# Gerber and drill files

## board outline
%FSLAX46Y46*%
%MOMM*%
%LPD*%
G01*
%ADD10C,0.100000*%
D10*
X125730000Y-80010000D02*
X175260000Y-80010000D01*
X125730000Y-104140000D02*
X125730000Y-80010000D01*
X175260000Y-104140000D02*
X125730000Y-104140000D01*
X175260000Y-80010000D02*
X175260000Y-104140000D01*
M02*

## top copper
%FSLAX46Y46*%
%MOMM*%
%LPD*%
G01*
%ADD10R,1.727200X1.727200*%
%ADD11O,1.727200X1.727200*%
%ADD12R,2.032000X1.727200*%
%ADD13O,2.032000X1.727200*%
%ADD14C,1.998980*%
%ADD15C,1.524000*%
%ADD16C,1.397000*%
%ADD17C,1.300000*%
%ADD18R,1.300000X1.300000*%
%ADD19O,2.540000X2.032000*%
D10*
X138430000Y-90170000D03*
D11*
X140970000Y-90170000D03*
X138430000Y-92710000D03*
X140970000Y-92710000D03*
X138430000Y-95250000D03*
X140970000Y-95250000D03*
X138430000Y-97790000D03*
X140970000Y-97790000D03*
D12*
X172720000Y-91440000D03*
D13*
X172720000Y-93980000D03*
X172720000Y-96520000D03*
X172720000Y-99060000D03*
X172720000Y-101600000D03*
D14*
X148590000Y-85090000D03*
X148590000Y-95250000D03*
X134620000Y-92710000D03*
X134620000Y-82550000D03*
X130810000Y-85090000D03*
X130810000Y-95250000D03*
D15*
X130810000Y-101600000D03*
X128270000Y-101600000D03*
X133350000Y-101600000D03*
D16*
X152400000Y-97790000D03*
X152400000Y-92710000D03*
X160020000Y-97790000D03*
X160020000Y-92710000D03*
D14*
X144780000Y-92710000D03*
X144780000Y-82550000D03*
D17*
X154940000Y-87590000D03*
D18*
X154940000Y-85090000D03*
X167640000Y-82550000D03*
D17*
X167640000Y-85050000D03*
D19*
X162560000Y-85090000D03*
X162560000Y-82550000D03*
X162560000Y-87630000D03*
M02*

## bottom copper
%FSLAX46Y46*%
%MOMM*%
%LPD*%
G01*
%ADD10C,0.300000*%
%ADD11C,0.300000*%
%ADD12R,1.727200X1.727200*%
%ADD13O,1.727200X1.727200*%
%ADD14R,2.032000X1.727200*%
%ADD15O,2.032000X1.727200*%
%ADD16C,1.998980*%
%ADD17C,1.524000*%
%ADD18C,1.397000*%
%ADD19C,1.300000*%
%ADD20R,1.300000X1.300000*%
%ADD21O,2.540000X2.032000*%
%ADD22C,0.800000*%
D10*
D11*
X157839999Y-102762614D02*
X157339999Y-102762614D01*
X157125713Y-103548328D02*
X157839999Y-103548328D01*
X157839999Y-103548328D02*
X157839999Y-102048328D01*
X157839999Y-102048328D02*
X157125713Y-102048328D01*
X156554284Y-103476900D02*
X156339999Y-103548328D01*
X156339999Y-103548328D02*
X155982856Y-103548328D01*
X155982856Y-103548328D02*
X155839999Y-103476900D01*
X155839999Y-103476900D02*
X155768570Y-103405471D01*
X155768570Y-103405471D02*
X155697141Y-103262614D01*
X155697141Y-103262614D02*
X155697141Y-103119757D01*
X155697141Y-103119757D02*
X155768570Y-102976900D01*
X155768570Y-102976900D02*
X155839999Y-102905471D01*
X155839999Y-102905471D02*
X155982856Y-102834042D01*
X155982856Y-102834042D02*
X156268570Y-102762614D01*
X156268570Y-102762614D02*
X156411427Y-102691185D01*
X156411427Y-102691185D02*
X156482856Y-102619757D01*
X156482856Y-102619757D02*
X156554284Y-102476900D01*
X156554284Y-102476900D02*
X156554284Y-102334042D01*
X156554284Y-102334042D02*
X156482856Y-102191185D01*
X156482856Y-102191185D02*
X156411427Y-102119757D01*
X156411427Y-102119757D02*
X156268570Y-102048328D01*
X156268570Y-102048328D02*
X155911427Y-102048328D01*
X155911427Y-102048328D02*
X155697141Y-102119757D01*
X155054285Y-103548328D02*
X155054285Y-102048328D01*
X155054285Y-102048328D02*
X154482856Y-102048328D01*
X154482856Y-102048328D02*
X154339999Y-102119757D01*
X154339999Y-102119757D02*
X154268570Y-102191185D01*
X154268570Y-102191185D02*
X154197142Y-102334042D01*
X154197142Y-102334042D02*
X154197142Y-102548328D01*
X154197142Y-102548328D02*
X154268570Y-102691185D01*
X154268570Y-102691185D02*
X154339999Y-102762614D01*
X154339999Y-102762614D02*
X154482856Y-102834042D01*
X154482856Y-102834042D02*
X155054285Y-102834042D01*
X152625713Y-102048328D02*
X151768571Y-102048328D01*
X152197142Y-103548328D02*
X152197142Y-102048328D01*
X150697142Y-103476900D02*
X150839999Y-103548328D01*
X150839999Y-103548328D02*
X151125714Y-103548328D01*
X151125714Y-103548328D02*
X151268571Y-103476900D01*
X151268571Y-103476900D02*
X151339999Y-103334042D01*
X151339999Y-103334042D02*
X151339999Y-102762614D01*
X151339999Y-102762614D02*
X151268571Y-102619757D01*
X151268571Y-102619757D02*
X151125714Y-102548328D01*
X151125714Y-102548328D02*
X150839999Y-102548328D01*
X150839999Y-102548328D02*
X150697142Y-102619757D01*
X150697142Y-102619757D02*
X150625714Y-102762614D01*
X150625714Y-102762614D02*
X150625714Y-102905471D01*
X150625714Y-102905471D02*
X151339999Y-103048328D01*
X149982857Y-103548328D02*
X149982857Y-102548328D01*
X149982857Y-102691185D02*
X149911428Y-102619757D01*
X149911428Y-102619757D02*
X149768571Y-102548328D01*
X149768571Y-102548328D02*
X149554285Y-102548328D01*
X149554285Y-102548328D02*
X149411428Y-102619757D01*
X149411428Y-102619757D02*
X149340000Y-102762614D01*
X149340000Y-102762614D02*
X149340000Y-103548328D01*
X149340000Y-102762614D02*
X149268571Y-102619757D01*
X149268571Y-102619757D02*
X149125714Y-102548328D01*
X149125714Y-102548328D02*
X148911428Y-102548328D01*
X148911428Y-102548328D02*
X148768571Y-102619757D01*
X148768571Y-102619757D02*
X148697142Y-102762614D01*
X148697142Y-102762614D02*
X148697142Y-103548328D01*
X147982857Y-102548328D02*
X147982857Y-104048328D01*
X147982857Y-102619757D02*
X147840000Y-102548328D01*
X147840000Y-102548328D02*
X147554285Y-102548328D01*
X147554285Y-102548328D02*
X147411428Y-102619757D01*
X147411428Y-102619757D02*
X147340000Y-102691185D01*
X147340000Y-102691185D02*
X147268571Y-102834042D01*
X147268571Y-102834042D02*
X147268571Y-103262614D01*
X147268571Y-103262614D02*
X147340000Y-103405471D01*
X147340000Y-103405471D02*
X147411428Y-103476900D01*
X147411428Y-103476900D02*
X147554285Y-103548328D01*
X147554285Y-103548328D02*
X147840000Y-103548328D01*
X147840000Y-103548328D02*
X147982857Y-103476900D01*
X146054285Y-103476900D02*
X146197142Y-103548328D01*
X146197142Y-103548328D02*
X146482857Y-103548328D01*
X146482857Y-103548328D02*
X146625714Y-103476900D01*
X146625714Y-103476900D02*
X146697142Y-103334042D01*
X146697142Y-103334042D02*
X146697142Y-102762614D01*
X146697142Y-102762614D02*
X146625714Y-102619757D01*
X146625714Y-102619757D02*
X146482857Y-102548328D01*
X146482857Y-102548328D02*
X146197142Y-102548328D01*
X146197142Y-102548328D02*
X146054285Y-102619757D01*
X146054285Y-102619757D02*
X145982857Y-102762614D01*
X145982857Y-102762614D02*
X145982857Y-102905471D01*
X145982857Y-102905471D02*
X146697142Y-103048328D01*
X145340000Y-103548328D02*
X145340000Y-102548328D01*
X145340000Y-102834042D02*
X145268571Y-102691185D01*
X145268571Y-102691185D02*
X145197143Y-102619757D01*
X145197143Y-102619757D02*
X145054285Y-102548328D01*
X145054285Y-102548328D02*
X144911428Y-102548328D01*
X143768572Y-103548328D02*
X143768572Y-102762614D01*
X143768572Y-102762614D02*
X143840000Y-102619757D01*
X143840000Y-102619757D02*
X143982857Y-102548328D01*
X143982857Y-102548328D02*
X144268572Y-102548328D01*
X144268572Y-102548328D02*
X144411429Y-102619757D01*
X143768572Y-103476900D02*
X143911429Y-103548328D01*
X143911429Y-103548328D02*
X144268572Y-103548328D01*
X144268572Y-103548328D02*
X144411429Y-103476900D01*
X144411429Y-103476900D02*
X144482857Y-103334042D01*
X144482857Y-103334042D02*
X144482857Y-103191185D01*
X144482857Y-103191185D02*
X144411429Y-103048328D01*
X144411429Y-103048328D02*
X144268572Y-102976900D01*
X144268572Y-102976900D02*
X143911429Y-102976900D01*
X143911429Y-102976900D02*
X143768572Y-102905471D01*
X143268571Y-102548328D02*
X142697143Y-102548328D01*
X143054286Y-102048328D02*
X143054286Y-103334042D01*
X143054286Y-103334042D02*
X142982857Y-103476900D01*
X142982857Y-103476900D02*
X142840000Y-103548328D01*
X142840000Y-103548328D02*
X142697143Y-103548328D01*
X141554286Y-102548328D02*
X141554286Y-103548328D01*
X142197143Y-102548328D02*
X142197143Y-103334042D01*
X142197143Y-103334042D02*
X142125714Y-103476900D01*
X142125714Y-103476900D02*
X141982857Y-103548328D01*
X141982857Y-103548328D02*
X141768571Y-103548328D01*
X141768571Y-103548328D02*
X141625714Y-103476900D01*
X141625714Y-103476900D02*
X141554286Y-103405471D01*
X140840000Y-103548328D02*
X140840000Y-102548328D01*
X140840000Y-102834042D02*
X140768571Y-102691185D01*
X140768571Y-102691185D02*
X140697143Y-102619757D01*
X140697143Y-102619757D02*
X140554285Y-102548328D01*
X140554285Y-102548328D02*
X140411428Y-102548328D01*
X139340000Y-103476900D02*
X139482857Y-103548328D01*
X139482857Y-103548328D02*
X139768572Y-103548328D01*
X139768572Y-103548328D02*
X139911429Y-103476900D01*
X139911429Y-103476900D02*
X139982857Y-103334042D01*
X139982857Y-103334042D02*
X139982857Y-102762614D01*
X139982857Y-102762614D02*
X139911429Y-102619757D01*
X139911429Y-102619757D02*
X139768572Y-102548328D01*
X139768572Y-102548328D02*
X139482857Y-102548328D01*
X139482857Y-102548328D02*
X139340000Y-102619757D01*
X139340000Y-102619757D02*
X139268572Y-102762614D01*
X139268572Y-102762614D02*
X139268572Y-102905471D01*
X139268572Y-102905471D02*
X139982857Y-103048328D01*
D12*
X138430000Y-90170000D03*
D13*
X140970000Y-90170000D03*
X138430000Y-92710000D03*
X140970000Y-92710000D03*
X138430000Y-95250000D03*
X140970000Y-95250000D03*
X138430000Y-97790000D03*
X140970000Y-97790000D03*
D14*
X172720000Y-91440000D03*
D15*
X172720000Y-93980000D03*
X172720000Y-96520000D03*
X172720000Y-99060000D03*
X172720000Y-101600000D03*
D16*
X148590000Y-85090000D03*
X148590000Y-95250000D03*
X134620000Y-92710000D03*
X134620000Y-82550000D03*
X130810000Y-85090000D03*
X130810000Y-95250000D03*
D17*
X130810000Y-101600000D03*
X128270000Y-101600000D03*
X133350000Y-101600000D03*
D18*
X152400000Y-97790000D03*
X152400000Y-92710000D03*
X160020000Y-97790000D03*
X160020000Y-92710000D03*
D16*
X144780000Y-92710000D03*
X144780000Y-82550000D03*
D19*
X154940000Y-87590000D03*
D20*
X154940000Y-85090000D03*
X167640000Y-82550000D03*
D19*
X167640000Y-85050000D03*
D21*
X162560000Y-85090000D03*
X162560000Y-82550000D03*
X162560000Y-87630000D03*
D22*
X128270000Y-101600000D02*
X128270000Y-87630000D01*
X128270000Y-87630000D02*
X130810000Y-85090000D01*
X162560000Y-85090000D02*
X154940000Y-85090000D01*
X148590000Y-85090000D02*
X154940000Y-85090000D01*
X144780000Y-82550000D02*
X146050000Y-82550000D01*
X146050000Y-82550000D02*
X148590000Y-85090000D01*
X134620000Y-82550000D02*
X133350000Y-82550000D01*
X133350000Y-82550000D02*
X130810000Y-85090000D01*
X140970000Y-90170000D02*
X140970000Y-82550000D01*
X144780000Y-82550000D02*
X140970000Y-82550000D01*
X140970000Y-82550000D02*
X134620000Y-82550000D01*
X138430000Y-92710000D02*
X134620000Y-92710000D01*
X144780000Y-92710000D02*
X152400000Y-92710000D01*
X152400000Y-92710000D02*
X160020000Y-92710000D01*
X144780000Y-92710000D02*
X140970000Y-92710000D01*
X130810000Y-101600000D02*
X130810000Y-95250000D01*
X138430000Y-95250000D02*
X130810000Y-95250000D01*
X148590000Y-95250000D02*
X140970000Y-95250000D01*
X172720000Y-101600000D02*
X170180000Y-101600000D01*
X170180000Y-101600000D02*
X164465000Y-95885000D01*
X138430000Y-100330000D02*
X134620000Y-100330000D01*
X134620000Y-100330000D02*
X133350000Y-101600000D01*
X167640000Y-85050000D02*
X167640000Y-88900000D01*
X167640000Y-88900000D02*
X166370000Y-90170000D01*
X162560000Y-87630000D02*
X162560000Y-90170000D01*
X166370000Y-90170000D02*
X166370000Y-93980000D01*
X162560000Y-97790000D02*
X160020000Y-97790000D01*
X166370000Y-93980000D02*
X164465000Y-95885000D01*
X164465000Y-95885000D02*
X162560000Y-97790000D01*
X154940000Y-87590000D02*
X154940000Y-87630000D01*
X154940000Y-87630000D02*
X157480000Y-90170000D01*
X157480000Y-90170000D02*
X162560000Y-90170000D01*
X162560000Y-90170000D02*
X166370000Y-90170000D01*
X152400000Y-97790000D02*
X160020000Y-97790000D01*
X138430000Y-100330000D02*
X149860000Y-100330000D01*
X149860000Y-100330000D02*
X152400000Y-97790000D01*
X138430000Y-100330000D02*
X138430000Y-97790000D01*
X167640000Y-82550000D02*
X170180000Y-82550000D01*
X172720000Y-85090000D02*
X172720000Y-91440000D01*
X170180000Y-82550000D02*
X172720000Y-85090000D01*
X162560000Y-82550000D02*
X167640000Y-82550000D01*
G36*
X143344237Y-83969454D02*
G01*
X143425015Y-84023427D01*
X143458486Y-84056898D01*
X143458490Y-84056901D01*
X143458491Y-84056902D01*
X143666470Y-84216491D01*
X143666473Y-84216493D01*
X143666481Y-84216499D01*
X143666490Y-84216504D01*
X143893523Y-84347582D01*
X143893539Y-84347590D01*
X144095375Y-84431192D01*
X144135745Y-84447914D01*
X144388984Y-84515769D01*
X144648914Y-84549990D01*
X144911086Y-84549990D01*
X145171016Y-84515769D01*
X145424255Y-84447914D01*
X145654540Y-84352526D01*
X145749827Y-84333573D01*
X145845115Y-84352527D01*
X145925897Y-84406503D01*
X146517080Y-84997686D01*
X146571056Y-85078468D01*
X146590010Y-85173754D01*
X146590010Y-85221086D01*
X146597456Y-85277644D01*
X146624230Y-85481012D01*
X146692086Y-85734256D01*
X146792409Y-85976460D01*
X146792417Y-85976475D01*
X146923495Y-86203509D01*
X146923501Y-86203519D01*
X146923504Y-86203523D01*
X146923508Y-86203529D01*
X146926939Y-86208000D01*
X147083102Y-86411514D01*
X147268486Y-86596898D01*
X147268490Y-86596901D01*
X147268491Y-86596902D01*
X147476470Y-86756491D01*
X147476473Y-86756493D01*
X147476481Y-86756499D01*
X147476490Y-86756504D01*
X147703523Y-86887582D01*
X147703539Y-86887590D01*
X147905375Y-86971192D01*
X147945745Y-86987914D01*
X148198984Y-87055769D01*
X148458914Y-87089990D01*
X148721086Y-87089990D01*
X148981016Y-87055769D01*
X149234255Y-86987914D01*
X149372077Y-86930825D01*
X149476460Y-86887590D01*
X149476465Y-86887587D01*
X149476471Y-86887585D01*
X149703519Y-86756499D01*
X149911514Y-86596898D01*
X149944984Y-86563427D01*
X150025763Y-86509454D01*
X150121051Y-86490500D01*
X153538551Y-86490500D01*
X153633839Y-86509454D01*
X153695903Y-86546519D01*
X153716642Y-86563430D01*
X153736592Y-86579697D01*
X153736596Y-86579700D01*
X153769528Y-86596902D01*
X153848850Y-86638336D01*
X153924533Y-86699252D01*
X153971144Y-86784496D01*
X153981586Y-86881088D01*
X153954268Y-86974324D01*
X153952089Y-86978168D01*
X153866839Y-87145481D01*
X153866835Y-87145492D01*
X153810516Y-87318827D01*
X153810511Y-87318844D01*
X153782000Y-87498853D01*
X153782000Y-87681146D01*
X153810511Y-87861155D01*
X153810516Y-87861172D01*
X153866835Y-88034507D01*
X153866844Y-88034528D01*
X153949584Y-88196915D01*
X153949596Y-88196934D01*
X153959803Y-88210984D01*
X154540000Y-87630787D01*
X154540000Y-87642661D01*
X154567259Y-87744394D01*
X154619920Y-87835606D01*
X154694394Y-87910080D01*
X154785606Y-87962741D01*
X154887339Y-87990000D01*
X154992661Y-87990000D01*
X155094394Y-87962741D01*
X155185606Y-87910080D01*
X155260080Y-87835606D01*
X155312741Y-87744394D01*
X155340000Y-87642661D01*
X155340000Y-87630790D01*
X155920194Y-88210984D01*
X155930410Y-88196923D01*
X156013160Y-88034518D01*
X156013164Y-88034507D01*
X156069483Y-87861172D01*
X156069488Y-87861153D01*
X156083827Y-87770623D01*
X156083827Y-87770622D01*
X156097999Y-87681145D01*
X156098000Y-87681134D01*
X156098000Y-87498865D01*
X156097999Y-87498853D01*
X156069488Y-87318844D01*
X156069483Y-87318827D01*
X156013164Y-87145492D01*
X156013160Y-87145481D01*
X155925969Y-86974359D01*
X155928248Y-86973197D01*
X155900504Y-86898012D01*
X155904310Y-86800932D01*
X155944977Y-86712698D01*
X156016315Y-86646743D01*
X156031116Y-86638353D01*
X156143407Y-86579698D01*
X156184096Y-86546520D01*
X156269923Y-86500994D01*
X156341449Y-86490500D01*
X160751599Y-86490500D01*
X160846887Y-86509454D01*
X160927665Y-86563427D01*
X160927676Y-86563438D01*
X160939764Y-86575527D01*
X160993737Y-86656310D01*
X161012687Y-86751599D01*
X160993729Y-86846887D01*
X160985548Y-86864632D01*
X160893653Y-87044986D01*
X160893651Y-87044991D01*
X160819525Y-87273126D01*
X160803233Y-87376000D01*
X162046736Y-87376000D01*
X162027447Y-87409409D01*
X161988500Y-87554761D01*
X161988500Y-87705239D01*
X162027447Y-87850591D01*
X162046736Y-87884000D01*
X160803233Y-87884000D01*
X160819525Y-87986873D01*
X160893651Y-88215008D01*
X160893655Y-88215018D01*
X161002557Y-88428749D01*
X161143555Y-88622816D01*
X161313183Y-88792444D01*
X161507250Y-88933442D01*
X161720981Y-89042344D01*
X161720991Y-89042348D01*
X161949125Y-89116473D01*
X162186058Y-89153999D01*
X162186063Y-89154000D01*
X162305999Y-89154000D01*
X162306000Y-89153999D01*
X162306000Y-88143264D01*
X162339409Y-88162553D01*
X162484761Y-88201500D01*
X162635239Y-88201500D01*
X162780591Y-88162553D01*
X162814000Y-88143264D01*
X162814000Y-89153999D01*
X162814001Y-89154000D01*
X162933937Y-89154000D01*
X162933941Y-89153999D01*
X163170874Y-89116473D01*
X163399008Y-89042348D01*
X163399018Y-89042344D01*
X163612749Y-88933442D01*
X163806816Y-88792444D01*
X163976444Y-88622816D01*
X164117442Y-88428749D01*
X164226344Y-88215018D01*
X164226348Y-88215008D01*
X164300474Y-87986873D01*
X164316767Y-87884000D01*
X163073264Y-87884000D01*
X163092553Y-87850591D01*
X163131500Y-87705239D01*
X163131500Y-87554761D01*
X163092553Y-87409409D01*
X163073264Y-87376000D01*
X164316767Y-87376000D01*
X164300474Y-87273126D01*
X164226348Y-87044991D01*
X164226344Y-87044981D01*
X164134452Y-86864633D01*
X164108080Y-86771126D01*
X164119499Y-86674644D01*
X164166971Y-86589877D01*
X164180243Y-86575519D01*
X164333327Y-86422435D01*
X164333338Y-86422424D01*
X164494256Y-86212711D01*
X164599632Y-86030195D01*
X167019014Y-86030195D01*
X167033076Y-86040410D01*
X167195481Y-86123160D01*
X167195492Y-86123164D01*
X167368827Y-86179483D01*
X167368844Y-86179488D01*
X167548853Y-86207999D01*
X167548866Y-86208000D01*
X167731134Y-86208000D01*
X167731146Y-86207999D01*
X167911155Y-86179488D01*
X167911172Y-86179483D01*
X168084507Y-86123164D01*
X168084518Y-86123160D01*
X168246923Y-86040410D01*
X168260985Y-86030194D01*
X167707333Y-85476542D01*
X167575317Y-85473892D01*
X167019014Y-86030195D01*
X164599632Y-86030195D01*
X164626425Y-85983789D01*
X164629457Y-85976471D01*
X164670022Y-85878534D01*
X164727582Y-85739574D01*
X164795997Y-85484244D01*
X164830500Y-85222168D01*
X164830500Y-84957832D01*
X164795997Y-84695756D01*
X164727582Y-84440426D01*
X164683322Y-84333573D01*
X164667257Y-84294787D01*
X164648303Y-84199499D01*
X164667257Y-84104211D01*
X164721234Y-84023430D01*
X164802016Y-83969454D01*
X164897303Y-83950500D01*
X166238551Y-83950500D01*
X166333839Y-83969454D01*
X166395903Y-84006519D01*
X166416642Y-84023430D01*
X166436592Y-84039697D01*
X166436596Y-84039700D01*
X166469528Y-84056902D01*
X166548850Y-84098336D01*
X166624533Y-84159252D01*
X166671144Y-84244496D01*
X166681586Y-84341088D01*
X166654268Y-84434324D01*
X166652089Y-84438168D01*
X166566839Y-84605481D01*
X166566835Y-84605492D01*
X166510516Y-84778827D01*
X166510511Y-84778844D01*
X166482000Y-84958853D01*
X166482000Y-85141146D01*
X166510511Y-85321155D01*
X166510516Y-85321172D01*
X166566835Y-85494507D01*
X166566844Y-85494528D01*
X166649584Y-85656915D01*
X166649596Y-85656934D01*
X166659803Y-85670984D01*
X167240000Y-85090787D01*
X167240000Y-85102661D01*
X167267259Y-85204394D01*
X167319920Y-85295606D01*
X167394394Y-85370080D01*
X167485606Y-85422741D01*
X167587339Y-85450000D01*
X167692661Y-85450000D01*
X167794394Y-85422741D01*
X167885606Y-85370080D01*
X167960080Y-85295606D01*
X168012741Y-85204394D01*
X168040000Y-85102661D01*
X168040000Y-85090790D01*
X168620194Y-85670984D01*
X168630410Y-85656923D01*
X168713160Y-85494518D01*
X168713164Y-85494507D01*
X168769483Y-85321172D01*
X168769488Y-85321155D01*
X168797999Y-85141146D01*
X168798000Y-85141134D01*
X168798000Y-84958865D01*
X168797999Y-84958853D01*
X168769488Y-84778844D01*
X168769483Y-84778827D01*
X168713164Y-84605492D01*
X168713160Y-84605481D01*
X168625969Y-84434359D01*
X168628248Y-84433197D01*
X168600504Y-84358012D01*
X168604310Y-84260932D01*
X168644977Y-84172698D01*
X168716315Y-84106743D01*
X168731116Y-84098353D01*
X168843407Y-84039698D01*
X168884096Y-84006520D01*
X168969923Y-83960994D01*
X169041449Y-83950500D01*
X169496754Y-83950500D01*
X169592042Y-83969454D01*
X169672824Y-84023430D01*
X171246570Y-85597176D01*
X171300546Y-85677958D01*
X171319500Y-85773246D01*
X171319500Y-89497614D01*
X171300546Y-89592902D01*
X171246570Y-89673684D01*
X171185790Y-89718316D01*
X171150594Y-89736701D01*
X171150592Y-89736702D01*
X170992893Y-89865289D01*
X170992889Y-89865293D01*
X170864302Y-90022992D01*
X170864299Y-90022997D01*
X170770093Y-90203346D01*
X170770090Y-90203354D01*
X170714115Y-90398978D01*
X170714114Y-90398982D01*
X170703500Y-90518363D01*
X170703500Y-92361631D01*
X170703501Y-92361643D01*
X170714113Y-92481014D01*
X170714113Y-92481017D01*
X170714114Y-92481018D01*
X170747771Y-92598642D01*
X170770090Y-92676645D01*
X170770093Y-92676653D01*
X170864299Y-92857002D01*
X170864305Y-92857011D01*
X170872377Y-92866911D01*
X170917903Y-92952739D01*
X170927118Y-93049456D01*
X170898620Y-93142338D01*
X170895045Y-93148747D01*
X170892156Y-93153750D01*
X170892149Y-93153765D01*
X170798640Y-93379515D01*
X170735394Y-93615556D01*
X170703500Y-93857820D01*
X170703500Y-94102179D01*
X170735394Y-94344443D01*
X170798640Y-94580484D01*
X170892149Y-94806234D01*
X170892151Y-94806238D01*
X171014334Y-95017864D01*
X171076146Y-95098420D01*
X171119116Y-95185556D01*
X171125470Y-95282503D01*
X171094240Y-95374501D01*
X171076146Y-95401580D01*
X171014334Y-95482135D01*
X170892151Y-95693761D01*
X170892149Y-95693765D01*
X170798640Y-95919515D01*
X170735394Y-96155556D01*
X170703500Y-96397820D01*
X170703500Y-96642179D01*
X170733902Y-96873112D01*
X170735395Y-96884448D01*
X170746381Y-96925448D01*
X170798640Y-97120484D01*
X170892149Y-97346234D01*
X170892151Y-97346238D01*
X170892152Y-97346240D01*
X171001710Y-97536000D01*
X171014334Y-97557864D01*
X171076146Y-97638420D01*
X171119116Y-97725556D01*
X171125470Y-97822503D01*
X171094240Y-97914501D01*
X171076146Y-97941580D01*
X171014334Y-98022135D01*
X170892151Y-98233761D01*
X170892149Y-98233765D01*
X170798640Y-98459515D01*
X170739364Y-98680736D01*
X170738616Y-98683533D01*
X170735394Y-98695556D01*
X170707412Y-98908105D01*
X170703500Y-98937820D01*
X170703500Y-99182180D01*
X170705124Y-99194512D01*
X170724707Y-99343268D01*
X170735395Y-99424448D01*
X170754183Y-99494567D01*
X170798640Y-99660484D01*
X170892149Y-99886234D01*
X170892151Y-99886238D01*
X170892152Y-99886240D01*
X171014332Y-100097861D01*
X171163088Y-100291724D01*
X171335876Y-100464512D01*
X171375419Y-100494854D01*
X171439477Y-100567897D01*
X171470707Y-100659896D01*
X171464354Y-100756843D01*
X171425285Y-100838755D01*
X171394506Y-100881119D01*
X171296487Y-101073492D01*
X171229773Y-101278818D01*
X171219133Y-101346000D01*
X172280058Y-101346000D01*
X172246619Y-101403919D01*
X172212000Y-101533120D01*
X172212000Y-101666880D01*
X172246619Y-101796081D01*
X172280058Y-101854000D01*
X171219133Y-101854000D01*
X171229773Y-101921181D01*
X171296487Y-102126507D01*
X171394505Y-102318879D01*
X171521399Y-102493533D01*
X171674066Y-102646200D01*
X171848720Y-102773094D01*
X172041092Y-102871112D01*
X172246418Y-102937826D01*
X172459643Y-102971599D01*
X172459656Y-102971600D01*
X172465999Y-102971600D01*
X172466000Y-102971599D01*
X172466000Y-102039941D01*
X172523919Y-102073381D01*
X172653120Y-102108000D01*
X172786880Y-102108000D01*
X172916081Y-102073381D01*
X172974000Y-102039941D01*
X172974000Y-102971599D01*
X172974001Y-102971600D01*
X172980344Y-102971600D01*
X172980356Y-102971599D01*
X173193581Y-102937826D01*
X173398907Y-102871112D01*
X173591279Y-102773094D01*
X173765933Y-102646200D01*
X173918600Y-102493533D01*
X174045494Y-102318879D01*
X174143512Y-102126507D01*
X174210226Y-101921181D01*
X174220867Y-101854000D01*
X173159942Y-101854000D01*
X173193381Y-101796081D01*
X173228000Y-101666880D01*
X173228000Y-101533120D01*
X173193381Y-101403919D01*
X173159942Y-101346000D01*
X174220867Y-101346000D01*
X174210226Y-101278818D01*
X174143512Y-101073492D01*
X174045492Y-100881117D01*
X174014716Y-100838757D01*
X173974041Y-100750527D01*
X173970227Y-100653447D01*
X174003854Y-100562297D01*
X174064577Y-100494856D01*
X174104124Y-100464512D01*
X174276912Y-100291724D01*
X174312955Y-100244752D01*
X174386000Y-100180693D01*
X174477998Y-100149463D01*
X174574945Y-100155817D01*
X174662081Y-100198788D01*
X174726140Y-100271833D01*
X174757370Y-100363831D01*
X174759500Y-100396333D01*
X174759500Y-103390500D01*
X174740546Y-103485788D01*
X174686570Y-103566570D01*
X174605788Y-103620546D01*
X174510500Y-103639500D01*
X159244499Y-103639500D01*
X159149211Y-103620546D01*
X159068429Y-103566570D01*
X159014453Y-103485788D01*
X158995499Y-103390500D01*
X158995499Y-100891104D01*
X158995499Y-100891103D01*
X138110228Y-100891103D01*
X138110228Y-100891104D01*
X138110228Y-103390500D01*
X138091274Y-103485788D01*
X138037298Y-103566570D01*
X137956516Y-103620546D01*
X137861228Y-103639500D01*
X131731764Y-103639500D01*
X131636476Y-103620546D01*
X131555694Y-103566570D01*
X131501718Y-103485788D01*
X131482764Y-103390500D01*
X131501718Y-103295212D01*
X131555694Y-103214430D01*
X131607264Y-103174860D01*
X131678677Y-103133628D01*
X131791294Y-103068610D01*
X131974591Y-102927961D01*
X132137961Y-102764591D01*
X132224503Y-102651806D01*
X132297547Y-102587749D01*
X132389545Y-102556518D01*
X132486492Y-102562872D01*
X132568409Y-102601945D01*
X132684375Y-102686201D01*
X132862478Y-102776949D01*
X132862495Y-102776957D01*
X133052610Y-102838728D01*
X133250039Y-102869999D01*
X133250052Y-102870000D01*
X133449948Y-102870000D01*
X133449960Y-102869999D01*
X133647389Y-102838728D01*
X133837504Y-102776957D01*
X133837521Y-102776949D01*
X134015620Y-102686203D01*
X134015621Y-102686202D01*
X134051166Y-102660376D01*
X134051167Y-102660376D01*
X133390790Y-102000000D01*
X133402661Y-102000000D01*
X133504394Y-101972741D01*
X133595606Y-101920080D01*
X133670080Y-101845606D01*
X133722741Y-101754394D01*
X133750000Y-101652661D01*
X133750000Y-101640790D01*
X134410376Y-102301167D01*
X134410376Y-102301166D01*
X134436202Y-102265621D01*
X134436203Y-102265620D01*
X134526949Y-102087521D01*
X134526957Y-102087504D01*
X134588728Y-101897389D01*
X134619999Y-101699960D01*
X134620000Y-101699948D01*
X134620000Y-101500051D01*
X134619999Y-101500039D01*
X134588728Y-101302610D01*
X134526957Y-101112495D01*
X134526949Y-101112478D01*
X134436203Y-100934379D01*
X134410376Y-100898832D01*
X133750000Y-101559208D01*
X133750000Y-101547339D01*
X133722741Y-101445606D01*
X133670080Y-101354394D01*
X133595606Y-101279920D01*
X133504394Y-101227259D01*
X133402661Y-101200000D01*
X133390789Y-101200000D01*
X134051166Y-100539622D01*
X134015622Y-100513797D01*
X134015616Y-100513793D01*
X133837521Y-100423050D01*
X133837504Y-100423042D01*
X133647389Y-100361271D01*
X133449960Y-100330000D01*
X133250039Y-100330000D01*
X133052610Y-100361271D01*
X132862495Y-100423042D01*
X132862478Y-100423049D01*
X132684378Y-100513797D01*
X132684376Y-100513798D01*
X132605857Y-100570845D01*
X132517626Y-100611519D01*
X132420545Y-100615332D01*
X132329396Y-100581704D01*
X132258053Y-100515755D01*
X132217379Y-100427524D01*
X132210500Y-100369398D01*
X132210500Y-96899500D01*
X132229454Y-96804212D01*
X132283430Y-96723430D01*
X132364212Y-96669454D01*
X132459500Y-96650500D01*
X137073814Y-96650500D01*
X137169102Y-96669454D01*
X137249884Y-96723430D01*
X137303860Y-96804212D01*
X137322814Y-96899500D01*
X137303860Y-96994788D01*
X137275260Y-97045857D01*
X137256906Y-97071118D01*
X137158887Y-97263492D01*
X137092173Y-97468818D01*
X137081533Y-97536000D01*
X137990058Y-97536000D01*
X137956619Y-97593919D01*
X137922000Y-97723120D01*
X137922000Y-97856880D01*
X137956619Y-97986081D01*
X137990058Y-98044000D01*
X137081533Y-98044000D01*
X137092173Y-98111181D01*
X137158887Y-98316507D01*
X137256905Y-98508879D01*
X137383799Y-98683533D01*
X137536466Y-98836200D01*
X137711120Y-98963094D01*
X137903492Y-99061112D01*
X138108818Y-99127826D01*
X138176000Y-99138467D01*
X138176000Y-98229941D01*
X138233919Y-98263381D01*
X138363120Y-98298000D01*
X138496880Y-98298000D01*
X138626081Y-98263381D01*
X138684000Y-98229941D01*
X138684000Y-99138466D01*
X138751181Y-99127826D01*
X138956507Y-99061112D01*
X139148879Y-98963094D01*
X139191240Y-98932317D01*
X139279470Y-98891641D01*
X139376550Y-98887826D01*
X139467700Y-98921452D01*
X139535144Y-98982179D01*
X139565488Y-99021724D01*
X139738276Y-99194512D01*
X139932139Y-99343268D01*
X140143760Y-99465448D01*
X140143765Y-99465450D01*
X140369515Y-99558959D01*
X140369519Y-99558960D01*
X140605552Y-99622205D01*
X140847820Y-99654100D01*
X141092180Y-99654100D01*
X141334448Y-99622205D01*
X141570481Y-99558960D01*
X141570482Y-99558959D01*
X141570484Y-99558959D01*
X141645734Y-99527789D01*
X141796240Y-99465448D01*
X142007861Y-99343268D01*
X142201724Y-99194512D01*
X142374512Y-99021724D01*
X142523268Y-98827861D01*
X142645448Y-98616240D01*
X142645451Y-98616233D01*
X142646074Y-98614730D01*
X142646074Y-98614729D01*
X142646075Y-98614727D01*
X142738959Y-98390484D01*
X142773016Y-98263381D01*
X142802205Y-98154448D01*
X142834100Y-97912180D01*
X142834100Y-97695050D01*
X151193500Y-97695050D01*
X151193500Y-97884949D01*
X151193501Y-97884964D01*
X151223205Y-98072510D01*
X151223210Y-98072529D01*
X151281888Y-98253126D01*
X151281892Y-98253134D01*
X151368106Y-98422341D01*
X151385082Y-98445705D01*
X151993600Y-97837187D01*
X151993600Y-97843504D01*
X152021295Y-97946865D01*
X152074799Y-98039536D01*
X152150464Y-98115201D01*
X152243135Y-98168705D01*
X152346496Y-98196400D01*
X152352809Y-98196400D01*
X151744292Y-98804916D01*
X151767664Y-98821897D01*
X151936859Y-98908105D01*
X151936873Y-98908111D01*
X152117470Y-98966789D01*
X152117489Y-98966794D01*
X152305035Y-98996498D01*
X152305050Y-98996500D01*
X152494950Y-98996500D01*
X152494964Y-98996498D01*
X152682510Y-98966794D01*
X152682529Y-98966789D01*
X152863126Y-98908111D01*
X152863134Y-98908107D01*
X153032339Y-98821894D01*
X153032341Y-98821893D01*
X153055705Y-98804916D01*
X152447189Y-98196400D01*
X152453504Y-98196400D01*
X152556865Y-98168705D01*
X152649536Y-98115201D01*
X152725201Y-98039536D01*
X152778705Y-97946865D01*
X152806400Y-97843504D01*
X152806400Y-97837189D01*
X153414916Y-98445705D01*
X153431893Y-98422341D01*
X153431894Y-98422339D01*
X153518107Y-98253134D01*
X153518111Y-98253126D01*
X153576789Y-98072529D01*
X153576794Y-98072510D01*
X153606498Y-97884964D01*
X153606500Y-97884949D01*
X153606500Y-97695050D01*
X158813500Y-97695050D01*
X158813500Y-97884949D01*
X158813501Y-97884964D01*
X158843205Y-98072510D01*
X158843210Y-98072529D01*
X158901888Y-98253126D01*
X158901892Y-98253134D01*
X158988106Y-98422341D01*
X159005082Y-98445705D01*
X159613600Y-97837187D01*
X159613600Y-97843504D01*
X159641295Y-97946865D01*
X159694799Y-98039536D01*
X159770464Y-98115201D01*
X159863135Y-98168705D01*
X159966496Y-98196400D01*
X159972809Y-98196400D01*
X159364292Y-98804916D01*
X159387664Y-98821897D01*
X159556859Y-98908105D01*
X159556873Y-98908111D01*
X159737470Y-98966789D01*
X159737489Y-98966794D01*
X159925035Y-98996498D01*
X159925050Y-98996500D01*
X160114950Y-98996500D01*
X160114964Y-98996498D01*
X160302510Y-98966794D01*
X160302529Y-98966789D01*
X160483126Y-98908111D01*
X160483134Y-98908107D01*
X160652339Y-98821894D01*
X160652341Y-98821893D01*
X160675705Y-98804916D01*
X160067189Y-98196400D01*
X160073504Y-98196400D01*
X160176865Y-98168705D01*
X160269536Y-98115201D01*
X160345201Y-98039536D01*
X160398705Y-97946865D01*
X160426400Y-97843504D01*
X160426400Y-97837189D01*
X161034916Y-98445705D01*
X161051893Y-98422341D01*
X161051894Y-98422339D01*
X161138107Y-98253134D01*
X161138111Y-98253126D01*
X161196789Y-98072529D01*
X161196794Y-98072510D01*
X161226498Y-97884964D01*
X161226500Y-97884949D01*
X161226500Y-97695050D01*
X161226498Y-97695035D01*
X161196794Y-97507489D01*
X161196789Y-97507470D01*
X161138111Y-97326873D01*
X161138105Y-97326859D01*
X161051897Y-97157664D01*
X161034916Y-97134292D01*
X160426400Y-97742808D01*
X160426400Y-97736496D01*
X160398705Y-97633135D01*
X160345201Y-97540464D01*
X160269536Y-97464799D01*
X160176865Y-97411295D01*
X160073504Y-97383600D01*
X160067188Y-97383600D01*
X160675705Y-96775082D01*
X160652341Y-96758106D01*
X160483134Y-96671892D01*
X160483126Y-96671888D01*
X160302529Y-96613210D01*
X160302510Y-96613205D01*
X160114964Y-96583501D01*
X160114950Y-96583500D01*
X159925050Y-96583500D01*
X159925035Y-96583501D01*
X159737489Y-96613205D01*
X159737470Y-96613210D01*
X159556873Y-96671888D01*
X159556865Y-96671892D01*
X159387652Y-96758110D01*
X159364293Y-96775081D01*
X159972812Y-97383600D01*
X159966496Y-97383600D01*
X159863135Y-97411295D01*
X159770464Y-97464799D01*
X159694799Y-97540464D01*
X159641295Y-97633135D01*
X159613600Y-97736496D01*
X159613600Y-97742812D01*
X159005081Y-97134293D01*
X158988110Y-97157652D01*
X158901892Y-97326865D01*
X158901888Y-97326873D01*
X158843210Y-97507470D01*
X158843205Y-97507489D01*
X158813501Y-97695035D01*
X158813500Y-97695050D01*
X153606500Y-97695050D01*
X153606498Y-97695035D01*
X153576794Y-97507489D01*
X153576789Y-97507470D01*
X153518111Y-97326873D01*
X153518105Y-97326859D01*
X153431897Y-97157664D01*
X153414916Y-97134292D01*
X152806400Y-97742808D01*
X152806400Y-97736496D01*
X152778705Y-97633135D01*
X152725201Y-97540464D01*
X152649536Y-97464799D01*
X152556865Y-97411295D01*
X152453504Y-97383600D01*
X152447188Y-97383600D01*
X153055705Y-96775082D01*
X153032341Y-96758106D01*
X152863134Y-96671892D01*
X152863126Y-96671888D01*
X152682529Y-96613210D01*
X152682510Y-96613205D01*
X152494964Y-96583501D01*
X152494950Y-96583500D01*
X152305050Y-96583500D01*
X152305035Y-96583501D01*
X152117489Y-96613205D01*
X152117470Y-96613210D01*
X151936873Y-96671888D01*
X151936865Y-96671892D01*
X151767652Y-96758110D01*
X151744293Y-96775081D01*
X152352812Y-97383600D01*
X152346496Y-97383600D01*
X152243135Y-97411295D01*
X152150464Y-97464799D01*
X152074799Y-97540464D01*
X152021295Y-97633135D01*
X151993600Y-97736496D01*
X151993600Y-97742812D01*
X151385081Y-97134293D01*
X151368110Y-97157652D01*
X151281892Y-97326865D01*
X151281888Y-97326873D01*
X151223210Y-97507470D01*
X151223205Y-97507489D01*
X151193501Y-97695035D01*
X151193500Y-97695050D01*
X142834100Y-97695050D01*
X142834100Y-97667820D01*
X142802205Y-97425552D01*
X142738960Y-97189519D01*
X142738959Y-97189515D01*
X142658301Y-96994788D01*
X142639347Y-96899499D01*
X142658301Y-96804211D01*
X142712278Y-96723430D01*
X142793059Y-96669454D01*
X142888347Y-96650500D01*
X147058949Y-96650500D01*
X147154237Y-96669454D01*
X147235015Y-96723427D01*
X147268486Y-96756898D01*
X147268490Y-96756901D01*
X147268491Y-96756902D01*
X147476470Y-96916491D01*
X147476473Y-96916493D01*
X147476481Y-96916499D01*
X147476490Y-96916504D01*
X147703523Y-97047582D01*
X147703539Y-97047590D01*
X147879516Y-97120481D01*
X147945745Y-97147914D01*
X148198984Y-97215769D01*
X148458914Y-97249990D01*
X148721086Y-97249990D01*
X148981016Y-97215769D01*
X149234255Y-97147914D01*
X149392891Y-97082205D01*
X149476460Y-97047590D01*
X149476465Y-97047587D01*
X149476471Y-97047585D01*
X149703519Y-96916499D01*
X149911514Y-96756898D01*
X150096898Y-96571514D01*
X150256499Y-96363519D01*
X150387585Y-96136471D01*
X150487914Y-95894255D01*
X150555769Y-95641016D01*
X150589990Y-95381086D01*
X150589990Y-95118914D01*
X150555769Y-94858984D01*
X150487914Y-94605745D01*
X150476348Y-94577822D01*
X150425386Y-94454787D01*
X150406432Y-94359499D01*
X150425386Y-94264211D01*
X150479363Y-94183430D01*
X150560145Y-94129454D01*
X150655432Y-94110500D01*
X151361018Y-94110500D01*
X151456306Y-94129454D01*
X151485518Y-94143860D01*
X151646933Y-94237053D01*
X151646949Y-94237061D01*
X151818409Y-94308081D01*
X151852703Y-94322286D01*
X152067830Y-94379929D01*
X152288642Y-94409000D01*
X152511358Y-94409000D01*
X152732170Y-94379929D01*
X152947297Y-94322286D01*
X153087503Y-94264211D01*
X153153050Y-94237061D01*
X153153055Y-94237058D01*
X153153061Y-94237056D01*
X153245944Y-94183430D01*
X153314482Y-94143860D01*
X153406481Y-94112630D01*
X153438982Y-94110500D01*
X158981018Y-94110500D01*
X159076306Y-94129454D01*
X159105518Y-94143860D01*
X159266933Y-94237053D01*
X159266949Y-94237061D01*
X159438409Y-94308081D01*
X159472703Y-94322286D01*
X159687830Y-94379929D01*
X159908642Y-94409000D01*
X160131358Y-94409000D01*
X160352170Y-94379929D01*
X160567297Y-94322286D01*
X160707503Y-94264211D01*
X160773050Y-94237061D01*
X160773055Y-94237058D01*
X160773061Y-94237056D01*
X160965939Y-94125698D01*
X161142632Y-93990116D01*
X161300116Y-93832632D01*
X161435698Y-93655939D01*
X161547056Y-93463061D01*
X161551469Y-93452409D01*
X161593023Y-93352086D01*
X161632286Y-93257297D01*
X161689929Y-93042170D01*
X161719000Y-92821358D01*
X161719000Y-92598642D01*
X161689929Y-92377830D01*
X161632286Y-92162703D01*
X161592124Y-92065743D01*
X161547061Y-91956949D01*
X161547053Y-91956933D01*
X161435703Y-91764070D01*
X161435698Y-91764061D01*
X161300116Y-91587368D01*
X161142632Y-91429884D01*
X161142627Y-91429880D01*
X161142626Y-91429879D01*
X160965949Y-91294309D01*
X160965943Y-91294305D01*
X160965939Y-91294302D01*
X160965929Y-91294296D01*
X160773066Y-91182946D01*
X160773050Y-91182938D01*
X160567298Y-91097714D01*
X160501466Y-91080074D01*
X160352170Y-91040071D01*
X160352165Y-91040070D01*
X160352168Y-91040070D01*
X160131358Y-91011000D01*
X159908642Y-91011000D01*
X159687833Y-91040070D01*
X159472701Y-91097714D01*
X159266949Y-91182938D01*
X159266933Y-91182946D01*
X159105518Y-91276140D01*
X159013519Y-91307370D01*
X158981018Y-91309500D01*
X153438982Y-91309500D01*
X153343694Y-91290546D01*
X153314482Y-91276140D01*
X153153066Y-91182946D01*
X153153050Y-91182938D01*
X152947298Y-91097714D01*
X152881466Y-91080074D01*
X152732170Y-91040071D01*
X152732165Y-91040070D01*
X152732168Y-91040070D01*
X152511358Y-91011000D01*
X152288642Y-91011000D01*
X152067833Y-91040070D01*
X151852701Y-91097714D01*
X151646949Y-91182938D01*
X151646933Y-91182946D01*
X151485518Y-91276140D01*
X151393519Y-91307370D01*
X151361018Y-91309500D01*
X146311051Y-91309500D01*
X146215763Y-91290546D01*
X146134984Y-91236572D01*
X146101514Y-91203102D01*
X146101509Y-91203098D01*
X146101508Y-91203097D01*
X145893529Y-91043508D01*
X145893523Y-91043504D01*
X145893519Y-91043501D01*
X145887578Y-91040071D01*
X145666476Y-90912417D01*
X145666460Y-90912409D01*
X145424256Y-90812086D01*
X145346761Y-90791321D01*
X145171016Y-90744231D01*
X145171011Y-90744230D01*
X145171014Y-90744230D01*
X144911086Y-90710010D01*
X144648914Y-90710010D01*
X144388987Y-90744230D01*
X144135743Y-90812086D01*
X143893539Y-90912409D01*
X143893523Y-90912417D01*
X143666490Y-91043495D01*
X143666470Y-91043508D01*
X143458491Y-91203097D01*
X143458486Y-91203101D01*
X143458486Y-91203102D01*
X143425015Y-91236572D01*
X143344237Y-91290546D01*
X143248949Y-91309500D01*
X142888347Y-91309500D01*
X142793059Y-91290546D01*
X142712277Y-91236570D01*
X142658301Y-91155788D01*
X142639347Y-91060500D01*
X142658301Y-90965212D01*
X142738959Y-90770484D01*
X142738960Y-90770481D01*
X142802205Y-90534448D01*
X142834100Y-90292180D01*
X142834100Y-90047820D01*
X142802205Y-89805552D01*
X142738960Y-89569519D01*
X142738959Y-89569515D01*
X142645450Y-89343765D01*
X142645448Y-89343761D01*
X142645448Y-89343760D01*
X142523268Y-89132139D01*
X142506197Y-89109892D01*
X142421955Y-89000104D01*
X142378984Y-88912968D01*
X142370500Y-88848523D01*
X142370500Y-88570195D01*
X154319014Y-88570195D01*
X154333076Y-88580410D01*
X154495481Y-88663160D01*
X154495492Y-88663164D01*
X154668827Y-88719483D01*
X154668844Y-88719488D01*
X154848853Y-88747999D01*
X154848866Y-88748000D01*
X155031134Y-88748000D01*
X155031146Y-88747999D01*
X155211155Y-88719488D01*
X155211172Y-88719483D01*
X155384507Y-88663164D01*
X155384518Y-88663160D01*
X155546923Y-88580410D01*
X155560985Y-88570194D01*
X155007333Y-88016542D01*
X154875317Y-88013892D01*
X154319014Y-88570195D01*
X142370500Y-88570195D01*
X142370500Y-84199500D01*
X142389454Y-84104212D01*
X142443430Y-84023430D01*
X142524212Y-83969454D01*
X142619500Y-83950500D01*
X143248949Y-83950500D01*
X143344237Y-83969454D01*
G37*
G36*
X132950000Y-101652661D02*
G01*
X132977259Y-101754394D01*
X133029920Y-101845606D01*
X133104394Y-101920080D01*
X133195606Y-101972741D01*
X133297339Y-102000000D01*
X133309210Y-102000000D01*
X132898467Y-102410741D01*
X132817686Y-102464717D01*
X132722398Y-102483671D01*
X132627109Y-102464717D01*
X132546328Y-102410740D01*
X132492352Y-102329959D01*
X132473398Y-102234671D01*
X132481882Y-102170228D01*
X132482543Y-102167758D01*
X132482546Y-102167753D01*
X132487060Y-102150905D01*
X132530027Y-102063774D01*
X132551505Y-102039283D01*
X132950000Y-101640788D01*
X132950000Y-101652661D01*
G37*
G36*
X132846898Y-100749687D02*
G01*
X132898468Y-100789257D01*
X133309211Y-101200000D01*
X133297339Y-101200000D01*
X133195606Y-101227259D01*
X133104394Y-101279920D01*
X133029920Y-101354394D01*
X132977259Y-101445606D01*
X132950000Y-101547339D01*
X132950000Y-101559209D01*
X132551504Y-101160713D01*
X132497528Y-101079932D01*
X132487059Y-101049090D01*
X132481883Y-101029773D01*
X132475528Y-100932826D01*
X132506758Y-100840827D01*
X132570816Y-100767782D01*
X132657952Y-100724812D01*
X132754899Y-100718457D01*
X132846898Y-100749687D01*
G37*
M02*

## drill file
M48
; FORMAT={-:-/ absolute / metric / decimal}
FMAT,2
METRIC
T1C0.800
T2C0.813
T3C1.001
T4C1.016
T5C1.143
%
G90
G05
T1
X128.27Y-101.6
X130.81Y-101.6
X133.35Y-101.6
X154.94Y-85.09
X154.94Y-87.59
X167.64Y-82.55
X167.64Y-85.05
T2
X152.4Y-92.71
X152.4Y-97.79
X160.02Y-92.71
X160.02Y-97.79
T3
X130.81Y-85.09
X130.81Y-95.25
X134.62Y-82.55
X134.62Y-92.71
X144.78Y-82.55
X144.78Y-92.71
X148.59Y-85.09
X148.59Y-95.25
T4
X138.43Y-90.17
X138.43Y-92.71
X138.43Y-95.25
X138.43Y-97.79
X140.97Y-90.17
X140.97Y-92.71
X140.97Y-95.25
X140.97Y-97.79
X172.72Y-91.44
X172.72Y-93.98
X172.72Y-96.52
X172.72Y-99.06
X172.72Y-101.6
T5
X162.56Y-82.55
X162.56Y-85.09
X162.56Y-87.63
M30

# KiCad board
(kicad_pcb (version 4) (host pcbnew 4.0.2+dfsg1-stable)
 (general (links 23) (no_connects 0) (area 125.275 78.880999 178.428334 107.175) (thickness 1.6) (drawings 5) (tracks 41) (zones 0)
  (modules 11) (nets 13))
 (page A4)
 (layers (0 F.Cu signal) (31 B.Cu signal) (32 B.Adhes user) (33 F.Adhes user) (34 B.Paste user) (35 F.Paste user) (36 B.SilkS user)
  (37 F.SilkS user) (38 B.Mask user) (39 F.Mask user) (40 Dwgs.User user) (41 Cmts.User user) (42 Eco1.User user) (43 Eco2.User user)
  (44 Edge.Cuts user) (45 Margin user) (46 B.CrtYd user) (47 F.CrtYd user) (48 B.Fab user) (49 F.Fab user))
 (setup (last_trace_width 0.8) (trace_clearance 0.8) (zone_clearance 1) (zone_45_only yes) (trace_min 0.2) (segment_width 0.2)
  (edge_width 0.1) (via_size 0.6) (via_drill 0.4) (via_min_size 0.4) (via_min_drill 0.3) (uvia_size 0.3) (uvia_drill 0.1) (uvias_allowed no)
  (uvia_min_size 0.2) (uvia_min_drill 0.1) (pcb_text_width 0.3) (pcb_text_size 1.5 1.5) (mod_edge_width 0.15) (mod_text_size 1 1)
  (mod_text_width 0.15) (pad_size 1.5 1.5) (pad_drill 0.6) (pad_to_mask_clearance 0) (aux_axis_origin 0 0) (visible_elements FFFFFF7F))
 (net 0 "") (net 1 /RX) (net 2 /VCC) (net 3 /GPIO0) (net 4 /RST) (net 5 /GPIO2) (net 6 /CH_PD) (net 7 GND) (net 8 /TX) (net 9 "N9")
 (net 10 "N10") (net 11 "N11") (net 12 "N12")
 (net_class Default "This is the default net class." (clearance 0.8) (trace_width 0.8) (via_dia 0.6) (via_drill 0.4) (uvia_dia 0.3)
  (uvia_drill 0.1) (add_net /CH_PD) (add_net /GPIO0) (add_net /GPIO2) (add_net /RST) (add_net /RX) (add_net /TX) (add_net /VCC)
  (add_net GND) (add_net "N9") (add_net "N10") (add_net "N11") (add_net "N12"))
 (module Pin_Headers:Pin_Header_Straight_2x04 (layer F.Cu) (at 138.43 90.17)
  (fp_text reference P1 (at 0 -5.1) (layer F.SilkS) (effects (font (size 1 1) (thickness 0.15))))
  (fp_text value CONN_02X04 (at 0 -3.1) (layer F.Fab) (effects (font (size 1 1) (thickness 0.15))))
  (pad 1 thru_hole rect (at 0 0) (size 1.7272 1.7272) (drill 1.016) (layers *.Cu *.Mask F.SilkS) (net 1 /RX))
  (pad 2 thru_hole oval (at 2.54 0) (size 1.7272 1.7272) (drill 1.016) (layers *.Cu *.Mask F.SilkS) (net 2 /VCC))
  (pad 3 thru_hole oval (at 0 2.54) (size 1.7272 1.7272) (drill 1.016) (layers *.Cu *.Mask F.SilkS) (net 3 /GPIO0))
  (pad 4 thru_hole oval (at 2.54 2.54) (size 1.7272 1.7272) (drill 1.016) (layers *.Cu *.Mask F.SilkS) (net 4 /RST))
  (pad 5 thru_hole oval (at 0 5.08) (size 1.7272 1.7272) (drill 1.016) (layers *.Cu *.Mask F.SilkS) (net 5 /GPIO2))
  (pad 6 thru_hole oval (at 2.54 5.08) (size 1.7272 1.7272) (drill 1.016) (layers *.Cu *.Mask F.SilkS) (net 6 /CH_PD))
  (pad 7 thru_hole oval (at 0 7.62) (size 1.7272 1.7272) (drill 1.016) (layers *.Cu *.Mask F.SilkS) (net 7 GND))
  (pad 8 thru_hole oval (at 2.54 7.62) (size 1.7272 1.7272) (drill 1.016) (layers *.Cu *.Mask F.SilkS) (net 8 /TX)))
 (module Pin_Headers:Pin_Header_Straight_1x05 (layer F.Cu) (at 172.72 91.44)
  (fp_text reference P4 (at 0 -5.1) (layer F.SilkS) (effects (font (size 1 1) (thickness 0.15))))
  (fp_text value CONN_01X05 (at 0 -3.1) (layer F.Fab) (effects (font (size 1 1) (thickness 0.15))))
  (pad 1 thru_hole rect (at 0 0) (size 2.032 1.7272) (drill 1.016) (layers *.Cu *.Mask F.SilkS) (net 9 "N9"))
  (pad 2 thru_hole oval (at 0 2.54) (size 2.032 1.7272) (drill 1.016) (layers *.Cu *.Mask F.SilkS) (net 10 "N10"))
  (pad 3 thru_hole oval (at 0 5.08) (size 2.032 1.7272) (drill 1.016) (layers *.Cu *.Mask F.SilkS) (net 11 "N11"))
  (pad 4 thru_hole oval (at 0 7.62) (size 2.032 1.7272) (drill 1.016) (layers *.Cu *.Mask F.SilkS) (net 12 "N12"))
  (pad 5 thru_hole oval (at 0 10.16) (size 2.032 1.7272) (drill 1.016) (layers *.Cu *.Mask F.SilkS) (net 7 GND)))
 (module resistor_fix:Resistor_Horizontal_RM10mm (layer F.Cu) (at 148.59 85.09 270)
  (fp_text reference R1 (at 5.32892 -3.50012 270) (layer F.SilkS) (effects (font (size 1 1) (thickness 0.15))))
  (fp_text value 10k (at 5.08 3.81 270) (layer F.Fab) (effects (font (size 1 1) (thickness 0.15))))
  (pad 1 thru_hole circle (at 0 0 270) (size 1.99898 1.99898) (drill 1.00076) (layers *.Cu *.SilkS *.Mask) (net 2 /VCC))
  (pad 2 thru_hole circle (at 10.16 0 270) (size 1.99898 1.99898) (drill 1.00076) (layers *.Cu *.SilkS *.Mask) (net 6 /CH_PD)))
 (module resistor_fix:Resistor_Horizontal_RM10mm (layer F.Cu) (at 134.62 92.71 90)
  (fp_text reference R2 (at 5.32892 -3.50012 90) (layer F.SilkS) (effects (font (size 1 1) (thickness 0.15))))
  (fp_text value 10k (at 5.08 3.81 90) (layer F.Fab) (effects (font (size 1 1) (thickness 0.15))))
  (pad 1 thru_hole circle (at 0 0 90) (size 1.99898 1.99898) (drill 1.00076) (layers *.Cu *.SilkS *.Mask) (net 3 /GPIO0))
  (pad 2 thru_hole circle (at 10.16 0 90) (size 1.99898 1.99898) (drill 1.00076) (layers *.Cu *.SilkS *.Mask) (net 2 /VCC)))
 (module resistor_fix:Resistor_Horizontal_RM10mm (layer F.Cu) (at 130.81 85.09 270)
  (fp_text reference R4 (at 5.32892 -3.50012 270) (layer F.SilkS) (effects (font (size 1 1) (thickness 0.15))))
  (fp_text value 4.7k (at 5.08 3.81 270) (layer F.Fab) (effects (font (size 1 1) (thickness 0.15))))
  (pad 1 thru_hole circle (at 0 0 270) (size 1.99898 1.99898) (drill 1.00076) (layers *.Cu *.SilkS *.Mask) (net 2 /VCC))
  (pad 2 thru_hole circle (at 10.16 0 270) (size 1.99898 1.99898) (drill 1.00076) (layers *.Cu *.SilkS *.Mask) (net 5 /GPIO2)))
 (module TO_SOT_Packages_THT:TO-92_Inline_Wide (layer F.Cu) (at 133.35 101.6 180)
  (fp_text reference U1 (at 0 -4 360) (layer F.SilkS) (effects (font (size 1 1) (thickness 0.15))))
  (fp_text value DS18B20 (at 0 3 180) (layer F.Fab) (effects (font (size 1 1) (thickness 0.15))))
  (pad 2 thru_hole circle (at 2.54 0 270) (size 1.524 1.524) (drill 0.8) (layers *.Cu *.Mask F.SilkS) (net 5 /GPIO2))
  (pad 3 thru_hole circle (at 5.08 0 270) (size 1.524 1.524) (drill 0.8) (layers *.Cu *.Mask F.SilkS) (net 2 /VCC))
  (pad 1 thru_hole circle (at 0 0 270) (size 1.524 1.524) (drill 0.8) (layers *.Cu *.Mask F.SilkS) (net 7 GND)))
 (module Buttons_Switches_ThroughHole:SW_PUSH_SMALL (layer F.Cu) (at 156.21 95.25 180)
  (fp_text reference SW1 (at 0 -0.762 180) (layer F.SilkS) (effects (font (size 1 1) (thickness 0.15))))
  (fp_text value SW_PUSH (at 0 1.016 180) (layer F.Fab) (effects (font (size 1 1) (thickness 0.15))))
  (pad 1 thru_hole circle (at 3.81 -2.54 180) (size 1.397 1.397) (drill 0.8128) (layers *.Cu *.Mask F.SilkS) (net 7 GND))
  (pad 2 thru_hole circle (at 3.81 2.54 180) (size 1.397 1.397) (drill 0.8128) (layers *.Cu *.Mask F.SilkS) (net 4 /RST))
  (pad 1 thru_hole circle (at -3.81 -2.54 180) (size 1.397 1.397) (drill 0.8128) (layers *.Cu *.Mask F.SilkS) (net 7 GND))
  (pad 2 thru_hole circle (at -3.81 2.54 180) (size 1.397 1.397) (drill 0.8128) (layers *.Cu *.Mask F.SilkS) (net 4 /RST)))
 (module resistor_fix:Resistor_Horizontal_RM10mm (layer F.Cu) (at 144.78 92.71 90)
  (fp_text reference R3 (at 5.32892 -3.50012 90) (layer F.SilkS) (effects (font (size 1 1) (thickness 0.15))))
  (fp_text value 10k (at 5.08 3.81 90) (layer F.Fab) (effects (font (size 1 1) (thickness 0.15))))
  (pad 1 thru_hole circle (at 0 0 90) (size 1.99898 1.99898) (drill 1.00076) (layers *.Cu *.SilkS *.Mask) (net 4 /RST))
  (pad 2 thru_hole circle (at 10.16 0 90) (size 1.99898 1.99898) (drill 1.00076) (layers *.Cu *.SilkS *.Mask) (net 2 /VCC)))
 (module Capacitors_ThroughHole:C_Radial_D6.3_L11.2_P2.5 (layer F.Cu) (at 154.94 85.09 270)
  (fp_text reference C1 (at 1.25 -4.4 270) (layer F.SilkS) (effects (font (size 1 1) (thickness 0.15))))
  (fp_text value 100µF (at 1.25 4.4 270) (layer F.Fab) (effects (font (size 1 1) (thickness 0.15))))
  (pad 2 thru_hole circle (at 2.5 0 270) (size 1.3 1.3) (drill 0.8) (layers *.Cu *.Mask F.SilkS) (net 7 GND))
  (pad 1 thru_hole rect (at 0 0 270) (size 1.3 1.3) (drill 0.8) (layers *.Cu *.Mask F.SilkS) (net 2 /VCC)))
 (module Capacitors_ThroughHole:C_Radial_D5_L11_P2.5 (layer F.Cu) (at 167.64 82.55 270)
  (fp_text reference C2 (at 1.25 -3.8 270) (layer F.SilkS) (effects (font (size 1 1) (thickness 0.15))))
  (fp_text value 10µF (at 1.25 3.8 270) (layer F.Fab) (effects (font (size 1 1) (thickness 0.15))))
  (pad 1 thru_hole rect (at 0 0 270) (size 1.3 1.3) (drill 0.8) (layers *.Cu *.Mask F.SilkS) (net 9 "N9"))
  (pad 2 thru_hole circle (at 2.5 0 270) (size 1.3 1.3) (drill 0.8) (layers *.Cu *.Mask F.SilkS) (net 7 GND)))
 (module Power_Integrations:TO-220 (layer F.Cu) (at 162.56 85.09 90)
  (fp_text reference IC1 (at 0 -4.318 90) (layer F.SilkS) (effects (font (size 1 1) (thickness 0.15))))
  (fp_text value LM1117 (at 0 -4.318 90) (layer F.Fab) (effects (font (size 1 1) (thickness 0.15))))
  (pad 2 thru_hole oval (at 0 0 90) (size 2.032 2.54) (drill 1.143) (layers *.Cu *.Mask F.SilkS) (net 2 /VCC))
  (pad 3 thru_hole oval (at 2.54 0 90) (size 2.032 2.54) (drill 1.143) (layers *.Cu *.Mask F.SilkS) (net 9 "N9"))
  (pad 1 thru_hole oval (at -2.54 0 90) (size 2.032 2.54) (drill 1.143) (layers *.Cu *.Mask F.SilkS) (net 7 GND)))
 (gr_line (start 125.73 80.01) (end 175.26 80.01) (angle 90) (layer Edge.Cuts) (width 0.1))
 (gr_line (start 125.73 104.14) (end 125.73 80.01) (angle 90) (layer Edge.Cuts) (width 0.1))
 (gr_line (start 175.26 104.14) (end 125.73 104.14) (angle 90) (layer Edge.Cuts) (width 0.1))
 (gr_line (start 175.26 80.01) (end 175.26 104.14) (angle 90) (layer Edge.Cuts) (width 0.1))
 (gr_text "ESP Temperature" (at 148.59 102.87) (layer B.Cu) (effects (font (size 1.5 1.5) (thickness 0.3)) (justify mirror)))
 (segment (start 128.27 101.6) (end 128.27 87.63) (width 0.8) (layer B.Cu) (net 2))
 (segment (start 128.27 87.63) (end 130.81 85.09) (width 0.8) (layer B.Cu) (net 2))
 (segment (start 162.56 85.09) (end 154.94 85.09) (width 0.8) (layer B.Cu) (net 2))
 (segment (start 148.59 85.09) (end 154.94 85.09) (width 0.8) (layer B.Cu) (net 2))
 (segment (start 144.78 82.55) (end 146.05 82.55) (width 0.8) (layer B.Cu) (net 2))
 (segment (start 146.05 82.55) (end 148.59 85.09) (width 0.8) (layer B.Cu) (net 2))
 (segment (start 134.62 82.55) (end 133.35 82.55) (width 0.8) (layer B.Cu) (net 2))
 (segment (start 133.35 82.55) (end 130.81 85.09) (width 0.8) (layer B.Cu) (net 2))
 (segment (start 140.97 90.17) (end 140.97 82.55) (width 0.8) (layer B.Cu) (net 2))
 (segment (start 144.78 82.55) (end 140.97 82.55) (width 0.8) (layer B.Cu) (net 2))
 (segment (start 140.97 82.55) (end 134.62 82.55) (width 0.8) (layer B.Cu) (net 2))
 (segment (start 138.43 92.71) (end 134.62 92.71) (width 0.8) (layer B.Cu) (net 3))
 (segment (start 144.78 92.71) (end 152.4 92.71) (width 0.8) (layer B.Cu) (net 4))
 (segment (start 152.4 92.71) (end 160.02 92.71) (width 0.8) (layer B.Cu) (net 4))
 (segment (start 144.78 92.71) (end 140.97 92.71) (width 0.8) (layer B.Cu) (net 4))
 (segment (start 130.81 101.6) (end 130.81 95.25) (width 0.8) (layer B.Cu) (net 5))
 (segment (start 138.43 95.25) (end 130.81 95.25) (width 0.8) (layer B.Cu) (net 5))
 (segment (start 148.59 95.25) (end 140.97 95.25) (width 0.8) (layer B.Cu) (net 6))
 (segment (start 172.72 101.6) (end 170.18 101.6) (width 0.8) (layer B.Cu) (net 7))
 (segment (start 170.18 101.6) (end 164.465 95.885) (width 0.8) (layer B.Cu) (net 7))
 (segment (start 138.43 100.33) (end 134.62 100.33) (width 0.8) (layer B.Cu) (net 7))
 (segment (start 134.62 100.33) (end 133.35 101.6) (width 0.8) (layer B.Cu) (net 7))
 (segment (start 167.64 85.05) (end 167.64 88.9) (width 0.8) (layer B.Cu) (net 7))
 (segment (start 167.64 88.9) (end 166.37 90.17) (width 0.8) (layer B.Cu) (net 7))
 (segment (start 162.56 87.63) (end 162.56 90.17) (width 0.8) (layer B.Cu) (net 7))
 (segment (start 166.37 90.17) (end 166.37 93.98) (width 0.8) (layer B.Cu) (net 7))
 (segment (start 162.56 97.79) (end 160.02 97.79) (width 0.8) (layer B.Cu) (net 7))
 (segment (start 166.37 93.98) (end 164.465 95.885) (width 0.8) (layer B.Cu) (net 7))
 (segment (start 164.465 95.885) (end 162.56 97.79) (width 0.8) (layer B.Cu) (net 7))
 (segment (start 154.94 87.59) (end 154.94 87.63) (width 0.8) (layer B.Cu) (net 7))
 (segment (start 154.94 87.63) (end 157.48 90.17) (width 0.8) (layer B.Cu) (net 7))
 (segment (start 157.48 90.17) (end 162.56 90.17) (width 0.8) (layer B.Cu) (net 7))
 (segment (start 162.56 90.17) (end 166.37 90.17) (width 0.8) (layer B.Cu) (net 7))
 (segment (start 152.4 97.79) (end 160.02 97.79) (width 0.8) (layer B.Cu) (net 7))
 (segment (start 138.43 100.33) (end 149.86 100.33) (width 0.8) (layer B.Cu) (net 7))
 (segment (start 149.86 100.33) (end 152.4 97.79) (width 0.8) (layer B.Cu) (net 7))
 (segment (start 138.43 100.33) (end 138.43 97.79) (width 0.8) (layer B.Cu) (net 7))
 (segment (start 167.64 82.55) (end 170.18 82.55) (width 0.8) (layer B.Cu) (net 9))
 (segment (start 172.72 85.09) (end 172.72 91.44) (width 0.8) (layer B.Cu) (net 9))
 (segment (start 170.18 82.55) (end 172.72 85.09) (width 0.8) (layer B.Cu) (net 9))
 (segment (start 162.56 82.55) (end 167.64 82.55) (width 0.8) (layer B.Cu) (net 9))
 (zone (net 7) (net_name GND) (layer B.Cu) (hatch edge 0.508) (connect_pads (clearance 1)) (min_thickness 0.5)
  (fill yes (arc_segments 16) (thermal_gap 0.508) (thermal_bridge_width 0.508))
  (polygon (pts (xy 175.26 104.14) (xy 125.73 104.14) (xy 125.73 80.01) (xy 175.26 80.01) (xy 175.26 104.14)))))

